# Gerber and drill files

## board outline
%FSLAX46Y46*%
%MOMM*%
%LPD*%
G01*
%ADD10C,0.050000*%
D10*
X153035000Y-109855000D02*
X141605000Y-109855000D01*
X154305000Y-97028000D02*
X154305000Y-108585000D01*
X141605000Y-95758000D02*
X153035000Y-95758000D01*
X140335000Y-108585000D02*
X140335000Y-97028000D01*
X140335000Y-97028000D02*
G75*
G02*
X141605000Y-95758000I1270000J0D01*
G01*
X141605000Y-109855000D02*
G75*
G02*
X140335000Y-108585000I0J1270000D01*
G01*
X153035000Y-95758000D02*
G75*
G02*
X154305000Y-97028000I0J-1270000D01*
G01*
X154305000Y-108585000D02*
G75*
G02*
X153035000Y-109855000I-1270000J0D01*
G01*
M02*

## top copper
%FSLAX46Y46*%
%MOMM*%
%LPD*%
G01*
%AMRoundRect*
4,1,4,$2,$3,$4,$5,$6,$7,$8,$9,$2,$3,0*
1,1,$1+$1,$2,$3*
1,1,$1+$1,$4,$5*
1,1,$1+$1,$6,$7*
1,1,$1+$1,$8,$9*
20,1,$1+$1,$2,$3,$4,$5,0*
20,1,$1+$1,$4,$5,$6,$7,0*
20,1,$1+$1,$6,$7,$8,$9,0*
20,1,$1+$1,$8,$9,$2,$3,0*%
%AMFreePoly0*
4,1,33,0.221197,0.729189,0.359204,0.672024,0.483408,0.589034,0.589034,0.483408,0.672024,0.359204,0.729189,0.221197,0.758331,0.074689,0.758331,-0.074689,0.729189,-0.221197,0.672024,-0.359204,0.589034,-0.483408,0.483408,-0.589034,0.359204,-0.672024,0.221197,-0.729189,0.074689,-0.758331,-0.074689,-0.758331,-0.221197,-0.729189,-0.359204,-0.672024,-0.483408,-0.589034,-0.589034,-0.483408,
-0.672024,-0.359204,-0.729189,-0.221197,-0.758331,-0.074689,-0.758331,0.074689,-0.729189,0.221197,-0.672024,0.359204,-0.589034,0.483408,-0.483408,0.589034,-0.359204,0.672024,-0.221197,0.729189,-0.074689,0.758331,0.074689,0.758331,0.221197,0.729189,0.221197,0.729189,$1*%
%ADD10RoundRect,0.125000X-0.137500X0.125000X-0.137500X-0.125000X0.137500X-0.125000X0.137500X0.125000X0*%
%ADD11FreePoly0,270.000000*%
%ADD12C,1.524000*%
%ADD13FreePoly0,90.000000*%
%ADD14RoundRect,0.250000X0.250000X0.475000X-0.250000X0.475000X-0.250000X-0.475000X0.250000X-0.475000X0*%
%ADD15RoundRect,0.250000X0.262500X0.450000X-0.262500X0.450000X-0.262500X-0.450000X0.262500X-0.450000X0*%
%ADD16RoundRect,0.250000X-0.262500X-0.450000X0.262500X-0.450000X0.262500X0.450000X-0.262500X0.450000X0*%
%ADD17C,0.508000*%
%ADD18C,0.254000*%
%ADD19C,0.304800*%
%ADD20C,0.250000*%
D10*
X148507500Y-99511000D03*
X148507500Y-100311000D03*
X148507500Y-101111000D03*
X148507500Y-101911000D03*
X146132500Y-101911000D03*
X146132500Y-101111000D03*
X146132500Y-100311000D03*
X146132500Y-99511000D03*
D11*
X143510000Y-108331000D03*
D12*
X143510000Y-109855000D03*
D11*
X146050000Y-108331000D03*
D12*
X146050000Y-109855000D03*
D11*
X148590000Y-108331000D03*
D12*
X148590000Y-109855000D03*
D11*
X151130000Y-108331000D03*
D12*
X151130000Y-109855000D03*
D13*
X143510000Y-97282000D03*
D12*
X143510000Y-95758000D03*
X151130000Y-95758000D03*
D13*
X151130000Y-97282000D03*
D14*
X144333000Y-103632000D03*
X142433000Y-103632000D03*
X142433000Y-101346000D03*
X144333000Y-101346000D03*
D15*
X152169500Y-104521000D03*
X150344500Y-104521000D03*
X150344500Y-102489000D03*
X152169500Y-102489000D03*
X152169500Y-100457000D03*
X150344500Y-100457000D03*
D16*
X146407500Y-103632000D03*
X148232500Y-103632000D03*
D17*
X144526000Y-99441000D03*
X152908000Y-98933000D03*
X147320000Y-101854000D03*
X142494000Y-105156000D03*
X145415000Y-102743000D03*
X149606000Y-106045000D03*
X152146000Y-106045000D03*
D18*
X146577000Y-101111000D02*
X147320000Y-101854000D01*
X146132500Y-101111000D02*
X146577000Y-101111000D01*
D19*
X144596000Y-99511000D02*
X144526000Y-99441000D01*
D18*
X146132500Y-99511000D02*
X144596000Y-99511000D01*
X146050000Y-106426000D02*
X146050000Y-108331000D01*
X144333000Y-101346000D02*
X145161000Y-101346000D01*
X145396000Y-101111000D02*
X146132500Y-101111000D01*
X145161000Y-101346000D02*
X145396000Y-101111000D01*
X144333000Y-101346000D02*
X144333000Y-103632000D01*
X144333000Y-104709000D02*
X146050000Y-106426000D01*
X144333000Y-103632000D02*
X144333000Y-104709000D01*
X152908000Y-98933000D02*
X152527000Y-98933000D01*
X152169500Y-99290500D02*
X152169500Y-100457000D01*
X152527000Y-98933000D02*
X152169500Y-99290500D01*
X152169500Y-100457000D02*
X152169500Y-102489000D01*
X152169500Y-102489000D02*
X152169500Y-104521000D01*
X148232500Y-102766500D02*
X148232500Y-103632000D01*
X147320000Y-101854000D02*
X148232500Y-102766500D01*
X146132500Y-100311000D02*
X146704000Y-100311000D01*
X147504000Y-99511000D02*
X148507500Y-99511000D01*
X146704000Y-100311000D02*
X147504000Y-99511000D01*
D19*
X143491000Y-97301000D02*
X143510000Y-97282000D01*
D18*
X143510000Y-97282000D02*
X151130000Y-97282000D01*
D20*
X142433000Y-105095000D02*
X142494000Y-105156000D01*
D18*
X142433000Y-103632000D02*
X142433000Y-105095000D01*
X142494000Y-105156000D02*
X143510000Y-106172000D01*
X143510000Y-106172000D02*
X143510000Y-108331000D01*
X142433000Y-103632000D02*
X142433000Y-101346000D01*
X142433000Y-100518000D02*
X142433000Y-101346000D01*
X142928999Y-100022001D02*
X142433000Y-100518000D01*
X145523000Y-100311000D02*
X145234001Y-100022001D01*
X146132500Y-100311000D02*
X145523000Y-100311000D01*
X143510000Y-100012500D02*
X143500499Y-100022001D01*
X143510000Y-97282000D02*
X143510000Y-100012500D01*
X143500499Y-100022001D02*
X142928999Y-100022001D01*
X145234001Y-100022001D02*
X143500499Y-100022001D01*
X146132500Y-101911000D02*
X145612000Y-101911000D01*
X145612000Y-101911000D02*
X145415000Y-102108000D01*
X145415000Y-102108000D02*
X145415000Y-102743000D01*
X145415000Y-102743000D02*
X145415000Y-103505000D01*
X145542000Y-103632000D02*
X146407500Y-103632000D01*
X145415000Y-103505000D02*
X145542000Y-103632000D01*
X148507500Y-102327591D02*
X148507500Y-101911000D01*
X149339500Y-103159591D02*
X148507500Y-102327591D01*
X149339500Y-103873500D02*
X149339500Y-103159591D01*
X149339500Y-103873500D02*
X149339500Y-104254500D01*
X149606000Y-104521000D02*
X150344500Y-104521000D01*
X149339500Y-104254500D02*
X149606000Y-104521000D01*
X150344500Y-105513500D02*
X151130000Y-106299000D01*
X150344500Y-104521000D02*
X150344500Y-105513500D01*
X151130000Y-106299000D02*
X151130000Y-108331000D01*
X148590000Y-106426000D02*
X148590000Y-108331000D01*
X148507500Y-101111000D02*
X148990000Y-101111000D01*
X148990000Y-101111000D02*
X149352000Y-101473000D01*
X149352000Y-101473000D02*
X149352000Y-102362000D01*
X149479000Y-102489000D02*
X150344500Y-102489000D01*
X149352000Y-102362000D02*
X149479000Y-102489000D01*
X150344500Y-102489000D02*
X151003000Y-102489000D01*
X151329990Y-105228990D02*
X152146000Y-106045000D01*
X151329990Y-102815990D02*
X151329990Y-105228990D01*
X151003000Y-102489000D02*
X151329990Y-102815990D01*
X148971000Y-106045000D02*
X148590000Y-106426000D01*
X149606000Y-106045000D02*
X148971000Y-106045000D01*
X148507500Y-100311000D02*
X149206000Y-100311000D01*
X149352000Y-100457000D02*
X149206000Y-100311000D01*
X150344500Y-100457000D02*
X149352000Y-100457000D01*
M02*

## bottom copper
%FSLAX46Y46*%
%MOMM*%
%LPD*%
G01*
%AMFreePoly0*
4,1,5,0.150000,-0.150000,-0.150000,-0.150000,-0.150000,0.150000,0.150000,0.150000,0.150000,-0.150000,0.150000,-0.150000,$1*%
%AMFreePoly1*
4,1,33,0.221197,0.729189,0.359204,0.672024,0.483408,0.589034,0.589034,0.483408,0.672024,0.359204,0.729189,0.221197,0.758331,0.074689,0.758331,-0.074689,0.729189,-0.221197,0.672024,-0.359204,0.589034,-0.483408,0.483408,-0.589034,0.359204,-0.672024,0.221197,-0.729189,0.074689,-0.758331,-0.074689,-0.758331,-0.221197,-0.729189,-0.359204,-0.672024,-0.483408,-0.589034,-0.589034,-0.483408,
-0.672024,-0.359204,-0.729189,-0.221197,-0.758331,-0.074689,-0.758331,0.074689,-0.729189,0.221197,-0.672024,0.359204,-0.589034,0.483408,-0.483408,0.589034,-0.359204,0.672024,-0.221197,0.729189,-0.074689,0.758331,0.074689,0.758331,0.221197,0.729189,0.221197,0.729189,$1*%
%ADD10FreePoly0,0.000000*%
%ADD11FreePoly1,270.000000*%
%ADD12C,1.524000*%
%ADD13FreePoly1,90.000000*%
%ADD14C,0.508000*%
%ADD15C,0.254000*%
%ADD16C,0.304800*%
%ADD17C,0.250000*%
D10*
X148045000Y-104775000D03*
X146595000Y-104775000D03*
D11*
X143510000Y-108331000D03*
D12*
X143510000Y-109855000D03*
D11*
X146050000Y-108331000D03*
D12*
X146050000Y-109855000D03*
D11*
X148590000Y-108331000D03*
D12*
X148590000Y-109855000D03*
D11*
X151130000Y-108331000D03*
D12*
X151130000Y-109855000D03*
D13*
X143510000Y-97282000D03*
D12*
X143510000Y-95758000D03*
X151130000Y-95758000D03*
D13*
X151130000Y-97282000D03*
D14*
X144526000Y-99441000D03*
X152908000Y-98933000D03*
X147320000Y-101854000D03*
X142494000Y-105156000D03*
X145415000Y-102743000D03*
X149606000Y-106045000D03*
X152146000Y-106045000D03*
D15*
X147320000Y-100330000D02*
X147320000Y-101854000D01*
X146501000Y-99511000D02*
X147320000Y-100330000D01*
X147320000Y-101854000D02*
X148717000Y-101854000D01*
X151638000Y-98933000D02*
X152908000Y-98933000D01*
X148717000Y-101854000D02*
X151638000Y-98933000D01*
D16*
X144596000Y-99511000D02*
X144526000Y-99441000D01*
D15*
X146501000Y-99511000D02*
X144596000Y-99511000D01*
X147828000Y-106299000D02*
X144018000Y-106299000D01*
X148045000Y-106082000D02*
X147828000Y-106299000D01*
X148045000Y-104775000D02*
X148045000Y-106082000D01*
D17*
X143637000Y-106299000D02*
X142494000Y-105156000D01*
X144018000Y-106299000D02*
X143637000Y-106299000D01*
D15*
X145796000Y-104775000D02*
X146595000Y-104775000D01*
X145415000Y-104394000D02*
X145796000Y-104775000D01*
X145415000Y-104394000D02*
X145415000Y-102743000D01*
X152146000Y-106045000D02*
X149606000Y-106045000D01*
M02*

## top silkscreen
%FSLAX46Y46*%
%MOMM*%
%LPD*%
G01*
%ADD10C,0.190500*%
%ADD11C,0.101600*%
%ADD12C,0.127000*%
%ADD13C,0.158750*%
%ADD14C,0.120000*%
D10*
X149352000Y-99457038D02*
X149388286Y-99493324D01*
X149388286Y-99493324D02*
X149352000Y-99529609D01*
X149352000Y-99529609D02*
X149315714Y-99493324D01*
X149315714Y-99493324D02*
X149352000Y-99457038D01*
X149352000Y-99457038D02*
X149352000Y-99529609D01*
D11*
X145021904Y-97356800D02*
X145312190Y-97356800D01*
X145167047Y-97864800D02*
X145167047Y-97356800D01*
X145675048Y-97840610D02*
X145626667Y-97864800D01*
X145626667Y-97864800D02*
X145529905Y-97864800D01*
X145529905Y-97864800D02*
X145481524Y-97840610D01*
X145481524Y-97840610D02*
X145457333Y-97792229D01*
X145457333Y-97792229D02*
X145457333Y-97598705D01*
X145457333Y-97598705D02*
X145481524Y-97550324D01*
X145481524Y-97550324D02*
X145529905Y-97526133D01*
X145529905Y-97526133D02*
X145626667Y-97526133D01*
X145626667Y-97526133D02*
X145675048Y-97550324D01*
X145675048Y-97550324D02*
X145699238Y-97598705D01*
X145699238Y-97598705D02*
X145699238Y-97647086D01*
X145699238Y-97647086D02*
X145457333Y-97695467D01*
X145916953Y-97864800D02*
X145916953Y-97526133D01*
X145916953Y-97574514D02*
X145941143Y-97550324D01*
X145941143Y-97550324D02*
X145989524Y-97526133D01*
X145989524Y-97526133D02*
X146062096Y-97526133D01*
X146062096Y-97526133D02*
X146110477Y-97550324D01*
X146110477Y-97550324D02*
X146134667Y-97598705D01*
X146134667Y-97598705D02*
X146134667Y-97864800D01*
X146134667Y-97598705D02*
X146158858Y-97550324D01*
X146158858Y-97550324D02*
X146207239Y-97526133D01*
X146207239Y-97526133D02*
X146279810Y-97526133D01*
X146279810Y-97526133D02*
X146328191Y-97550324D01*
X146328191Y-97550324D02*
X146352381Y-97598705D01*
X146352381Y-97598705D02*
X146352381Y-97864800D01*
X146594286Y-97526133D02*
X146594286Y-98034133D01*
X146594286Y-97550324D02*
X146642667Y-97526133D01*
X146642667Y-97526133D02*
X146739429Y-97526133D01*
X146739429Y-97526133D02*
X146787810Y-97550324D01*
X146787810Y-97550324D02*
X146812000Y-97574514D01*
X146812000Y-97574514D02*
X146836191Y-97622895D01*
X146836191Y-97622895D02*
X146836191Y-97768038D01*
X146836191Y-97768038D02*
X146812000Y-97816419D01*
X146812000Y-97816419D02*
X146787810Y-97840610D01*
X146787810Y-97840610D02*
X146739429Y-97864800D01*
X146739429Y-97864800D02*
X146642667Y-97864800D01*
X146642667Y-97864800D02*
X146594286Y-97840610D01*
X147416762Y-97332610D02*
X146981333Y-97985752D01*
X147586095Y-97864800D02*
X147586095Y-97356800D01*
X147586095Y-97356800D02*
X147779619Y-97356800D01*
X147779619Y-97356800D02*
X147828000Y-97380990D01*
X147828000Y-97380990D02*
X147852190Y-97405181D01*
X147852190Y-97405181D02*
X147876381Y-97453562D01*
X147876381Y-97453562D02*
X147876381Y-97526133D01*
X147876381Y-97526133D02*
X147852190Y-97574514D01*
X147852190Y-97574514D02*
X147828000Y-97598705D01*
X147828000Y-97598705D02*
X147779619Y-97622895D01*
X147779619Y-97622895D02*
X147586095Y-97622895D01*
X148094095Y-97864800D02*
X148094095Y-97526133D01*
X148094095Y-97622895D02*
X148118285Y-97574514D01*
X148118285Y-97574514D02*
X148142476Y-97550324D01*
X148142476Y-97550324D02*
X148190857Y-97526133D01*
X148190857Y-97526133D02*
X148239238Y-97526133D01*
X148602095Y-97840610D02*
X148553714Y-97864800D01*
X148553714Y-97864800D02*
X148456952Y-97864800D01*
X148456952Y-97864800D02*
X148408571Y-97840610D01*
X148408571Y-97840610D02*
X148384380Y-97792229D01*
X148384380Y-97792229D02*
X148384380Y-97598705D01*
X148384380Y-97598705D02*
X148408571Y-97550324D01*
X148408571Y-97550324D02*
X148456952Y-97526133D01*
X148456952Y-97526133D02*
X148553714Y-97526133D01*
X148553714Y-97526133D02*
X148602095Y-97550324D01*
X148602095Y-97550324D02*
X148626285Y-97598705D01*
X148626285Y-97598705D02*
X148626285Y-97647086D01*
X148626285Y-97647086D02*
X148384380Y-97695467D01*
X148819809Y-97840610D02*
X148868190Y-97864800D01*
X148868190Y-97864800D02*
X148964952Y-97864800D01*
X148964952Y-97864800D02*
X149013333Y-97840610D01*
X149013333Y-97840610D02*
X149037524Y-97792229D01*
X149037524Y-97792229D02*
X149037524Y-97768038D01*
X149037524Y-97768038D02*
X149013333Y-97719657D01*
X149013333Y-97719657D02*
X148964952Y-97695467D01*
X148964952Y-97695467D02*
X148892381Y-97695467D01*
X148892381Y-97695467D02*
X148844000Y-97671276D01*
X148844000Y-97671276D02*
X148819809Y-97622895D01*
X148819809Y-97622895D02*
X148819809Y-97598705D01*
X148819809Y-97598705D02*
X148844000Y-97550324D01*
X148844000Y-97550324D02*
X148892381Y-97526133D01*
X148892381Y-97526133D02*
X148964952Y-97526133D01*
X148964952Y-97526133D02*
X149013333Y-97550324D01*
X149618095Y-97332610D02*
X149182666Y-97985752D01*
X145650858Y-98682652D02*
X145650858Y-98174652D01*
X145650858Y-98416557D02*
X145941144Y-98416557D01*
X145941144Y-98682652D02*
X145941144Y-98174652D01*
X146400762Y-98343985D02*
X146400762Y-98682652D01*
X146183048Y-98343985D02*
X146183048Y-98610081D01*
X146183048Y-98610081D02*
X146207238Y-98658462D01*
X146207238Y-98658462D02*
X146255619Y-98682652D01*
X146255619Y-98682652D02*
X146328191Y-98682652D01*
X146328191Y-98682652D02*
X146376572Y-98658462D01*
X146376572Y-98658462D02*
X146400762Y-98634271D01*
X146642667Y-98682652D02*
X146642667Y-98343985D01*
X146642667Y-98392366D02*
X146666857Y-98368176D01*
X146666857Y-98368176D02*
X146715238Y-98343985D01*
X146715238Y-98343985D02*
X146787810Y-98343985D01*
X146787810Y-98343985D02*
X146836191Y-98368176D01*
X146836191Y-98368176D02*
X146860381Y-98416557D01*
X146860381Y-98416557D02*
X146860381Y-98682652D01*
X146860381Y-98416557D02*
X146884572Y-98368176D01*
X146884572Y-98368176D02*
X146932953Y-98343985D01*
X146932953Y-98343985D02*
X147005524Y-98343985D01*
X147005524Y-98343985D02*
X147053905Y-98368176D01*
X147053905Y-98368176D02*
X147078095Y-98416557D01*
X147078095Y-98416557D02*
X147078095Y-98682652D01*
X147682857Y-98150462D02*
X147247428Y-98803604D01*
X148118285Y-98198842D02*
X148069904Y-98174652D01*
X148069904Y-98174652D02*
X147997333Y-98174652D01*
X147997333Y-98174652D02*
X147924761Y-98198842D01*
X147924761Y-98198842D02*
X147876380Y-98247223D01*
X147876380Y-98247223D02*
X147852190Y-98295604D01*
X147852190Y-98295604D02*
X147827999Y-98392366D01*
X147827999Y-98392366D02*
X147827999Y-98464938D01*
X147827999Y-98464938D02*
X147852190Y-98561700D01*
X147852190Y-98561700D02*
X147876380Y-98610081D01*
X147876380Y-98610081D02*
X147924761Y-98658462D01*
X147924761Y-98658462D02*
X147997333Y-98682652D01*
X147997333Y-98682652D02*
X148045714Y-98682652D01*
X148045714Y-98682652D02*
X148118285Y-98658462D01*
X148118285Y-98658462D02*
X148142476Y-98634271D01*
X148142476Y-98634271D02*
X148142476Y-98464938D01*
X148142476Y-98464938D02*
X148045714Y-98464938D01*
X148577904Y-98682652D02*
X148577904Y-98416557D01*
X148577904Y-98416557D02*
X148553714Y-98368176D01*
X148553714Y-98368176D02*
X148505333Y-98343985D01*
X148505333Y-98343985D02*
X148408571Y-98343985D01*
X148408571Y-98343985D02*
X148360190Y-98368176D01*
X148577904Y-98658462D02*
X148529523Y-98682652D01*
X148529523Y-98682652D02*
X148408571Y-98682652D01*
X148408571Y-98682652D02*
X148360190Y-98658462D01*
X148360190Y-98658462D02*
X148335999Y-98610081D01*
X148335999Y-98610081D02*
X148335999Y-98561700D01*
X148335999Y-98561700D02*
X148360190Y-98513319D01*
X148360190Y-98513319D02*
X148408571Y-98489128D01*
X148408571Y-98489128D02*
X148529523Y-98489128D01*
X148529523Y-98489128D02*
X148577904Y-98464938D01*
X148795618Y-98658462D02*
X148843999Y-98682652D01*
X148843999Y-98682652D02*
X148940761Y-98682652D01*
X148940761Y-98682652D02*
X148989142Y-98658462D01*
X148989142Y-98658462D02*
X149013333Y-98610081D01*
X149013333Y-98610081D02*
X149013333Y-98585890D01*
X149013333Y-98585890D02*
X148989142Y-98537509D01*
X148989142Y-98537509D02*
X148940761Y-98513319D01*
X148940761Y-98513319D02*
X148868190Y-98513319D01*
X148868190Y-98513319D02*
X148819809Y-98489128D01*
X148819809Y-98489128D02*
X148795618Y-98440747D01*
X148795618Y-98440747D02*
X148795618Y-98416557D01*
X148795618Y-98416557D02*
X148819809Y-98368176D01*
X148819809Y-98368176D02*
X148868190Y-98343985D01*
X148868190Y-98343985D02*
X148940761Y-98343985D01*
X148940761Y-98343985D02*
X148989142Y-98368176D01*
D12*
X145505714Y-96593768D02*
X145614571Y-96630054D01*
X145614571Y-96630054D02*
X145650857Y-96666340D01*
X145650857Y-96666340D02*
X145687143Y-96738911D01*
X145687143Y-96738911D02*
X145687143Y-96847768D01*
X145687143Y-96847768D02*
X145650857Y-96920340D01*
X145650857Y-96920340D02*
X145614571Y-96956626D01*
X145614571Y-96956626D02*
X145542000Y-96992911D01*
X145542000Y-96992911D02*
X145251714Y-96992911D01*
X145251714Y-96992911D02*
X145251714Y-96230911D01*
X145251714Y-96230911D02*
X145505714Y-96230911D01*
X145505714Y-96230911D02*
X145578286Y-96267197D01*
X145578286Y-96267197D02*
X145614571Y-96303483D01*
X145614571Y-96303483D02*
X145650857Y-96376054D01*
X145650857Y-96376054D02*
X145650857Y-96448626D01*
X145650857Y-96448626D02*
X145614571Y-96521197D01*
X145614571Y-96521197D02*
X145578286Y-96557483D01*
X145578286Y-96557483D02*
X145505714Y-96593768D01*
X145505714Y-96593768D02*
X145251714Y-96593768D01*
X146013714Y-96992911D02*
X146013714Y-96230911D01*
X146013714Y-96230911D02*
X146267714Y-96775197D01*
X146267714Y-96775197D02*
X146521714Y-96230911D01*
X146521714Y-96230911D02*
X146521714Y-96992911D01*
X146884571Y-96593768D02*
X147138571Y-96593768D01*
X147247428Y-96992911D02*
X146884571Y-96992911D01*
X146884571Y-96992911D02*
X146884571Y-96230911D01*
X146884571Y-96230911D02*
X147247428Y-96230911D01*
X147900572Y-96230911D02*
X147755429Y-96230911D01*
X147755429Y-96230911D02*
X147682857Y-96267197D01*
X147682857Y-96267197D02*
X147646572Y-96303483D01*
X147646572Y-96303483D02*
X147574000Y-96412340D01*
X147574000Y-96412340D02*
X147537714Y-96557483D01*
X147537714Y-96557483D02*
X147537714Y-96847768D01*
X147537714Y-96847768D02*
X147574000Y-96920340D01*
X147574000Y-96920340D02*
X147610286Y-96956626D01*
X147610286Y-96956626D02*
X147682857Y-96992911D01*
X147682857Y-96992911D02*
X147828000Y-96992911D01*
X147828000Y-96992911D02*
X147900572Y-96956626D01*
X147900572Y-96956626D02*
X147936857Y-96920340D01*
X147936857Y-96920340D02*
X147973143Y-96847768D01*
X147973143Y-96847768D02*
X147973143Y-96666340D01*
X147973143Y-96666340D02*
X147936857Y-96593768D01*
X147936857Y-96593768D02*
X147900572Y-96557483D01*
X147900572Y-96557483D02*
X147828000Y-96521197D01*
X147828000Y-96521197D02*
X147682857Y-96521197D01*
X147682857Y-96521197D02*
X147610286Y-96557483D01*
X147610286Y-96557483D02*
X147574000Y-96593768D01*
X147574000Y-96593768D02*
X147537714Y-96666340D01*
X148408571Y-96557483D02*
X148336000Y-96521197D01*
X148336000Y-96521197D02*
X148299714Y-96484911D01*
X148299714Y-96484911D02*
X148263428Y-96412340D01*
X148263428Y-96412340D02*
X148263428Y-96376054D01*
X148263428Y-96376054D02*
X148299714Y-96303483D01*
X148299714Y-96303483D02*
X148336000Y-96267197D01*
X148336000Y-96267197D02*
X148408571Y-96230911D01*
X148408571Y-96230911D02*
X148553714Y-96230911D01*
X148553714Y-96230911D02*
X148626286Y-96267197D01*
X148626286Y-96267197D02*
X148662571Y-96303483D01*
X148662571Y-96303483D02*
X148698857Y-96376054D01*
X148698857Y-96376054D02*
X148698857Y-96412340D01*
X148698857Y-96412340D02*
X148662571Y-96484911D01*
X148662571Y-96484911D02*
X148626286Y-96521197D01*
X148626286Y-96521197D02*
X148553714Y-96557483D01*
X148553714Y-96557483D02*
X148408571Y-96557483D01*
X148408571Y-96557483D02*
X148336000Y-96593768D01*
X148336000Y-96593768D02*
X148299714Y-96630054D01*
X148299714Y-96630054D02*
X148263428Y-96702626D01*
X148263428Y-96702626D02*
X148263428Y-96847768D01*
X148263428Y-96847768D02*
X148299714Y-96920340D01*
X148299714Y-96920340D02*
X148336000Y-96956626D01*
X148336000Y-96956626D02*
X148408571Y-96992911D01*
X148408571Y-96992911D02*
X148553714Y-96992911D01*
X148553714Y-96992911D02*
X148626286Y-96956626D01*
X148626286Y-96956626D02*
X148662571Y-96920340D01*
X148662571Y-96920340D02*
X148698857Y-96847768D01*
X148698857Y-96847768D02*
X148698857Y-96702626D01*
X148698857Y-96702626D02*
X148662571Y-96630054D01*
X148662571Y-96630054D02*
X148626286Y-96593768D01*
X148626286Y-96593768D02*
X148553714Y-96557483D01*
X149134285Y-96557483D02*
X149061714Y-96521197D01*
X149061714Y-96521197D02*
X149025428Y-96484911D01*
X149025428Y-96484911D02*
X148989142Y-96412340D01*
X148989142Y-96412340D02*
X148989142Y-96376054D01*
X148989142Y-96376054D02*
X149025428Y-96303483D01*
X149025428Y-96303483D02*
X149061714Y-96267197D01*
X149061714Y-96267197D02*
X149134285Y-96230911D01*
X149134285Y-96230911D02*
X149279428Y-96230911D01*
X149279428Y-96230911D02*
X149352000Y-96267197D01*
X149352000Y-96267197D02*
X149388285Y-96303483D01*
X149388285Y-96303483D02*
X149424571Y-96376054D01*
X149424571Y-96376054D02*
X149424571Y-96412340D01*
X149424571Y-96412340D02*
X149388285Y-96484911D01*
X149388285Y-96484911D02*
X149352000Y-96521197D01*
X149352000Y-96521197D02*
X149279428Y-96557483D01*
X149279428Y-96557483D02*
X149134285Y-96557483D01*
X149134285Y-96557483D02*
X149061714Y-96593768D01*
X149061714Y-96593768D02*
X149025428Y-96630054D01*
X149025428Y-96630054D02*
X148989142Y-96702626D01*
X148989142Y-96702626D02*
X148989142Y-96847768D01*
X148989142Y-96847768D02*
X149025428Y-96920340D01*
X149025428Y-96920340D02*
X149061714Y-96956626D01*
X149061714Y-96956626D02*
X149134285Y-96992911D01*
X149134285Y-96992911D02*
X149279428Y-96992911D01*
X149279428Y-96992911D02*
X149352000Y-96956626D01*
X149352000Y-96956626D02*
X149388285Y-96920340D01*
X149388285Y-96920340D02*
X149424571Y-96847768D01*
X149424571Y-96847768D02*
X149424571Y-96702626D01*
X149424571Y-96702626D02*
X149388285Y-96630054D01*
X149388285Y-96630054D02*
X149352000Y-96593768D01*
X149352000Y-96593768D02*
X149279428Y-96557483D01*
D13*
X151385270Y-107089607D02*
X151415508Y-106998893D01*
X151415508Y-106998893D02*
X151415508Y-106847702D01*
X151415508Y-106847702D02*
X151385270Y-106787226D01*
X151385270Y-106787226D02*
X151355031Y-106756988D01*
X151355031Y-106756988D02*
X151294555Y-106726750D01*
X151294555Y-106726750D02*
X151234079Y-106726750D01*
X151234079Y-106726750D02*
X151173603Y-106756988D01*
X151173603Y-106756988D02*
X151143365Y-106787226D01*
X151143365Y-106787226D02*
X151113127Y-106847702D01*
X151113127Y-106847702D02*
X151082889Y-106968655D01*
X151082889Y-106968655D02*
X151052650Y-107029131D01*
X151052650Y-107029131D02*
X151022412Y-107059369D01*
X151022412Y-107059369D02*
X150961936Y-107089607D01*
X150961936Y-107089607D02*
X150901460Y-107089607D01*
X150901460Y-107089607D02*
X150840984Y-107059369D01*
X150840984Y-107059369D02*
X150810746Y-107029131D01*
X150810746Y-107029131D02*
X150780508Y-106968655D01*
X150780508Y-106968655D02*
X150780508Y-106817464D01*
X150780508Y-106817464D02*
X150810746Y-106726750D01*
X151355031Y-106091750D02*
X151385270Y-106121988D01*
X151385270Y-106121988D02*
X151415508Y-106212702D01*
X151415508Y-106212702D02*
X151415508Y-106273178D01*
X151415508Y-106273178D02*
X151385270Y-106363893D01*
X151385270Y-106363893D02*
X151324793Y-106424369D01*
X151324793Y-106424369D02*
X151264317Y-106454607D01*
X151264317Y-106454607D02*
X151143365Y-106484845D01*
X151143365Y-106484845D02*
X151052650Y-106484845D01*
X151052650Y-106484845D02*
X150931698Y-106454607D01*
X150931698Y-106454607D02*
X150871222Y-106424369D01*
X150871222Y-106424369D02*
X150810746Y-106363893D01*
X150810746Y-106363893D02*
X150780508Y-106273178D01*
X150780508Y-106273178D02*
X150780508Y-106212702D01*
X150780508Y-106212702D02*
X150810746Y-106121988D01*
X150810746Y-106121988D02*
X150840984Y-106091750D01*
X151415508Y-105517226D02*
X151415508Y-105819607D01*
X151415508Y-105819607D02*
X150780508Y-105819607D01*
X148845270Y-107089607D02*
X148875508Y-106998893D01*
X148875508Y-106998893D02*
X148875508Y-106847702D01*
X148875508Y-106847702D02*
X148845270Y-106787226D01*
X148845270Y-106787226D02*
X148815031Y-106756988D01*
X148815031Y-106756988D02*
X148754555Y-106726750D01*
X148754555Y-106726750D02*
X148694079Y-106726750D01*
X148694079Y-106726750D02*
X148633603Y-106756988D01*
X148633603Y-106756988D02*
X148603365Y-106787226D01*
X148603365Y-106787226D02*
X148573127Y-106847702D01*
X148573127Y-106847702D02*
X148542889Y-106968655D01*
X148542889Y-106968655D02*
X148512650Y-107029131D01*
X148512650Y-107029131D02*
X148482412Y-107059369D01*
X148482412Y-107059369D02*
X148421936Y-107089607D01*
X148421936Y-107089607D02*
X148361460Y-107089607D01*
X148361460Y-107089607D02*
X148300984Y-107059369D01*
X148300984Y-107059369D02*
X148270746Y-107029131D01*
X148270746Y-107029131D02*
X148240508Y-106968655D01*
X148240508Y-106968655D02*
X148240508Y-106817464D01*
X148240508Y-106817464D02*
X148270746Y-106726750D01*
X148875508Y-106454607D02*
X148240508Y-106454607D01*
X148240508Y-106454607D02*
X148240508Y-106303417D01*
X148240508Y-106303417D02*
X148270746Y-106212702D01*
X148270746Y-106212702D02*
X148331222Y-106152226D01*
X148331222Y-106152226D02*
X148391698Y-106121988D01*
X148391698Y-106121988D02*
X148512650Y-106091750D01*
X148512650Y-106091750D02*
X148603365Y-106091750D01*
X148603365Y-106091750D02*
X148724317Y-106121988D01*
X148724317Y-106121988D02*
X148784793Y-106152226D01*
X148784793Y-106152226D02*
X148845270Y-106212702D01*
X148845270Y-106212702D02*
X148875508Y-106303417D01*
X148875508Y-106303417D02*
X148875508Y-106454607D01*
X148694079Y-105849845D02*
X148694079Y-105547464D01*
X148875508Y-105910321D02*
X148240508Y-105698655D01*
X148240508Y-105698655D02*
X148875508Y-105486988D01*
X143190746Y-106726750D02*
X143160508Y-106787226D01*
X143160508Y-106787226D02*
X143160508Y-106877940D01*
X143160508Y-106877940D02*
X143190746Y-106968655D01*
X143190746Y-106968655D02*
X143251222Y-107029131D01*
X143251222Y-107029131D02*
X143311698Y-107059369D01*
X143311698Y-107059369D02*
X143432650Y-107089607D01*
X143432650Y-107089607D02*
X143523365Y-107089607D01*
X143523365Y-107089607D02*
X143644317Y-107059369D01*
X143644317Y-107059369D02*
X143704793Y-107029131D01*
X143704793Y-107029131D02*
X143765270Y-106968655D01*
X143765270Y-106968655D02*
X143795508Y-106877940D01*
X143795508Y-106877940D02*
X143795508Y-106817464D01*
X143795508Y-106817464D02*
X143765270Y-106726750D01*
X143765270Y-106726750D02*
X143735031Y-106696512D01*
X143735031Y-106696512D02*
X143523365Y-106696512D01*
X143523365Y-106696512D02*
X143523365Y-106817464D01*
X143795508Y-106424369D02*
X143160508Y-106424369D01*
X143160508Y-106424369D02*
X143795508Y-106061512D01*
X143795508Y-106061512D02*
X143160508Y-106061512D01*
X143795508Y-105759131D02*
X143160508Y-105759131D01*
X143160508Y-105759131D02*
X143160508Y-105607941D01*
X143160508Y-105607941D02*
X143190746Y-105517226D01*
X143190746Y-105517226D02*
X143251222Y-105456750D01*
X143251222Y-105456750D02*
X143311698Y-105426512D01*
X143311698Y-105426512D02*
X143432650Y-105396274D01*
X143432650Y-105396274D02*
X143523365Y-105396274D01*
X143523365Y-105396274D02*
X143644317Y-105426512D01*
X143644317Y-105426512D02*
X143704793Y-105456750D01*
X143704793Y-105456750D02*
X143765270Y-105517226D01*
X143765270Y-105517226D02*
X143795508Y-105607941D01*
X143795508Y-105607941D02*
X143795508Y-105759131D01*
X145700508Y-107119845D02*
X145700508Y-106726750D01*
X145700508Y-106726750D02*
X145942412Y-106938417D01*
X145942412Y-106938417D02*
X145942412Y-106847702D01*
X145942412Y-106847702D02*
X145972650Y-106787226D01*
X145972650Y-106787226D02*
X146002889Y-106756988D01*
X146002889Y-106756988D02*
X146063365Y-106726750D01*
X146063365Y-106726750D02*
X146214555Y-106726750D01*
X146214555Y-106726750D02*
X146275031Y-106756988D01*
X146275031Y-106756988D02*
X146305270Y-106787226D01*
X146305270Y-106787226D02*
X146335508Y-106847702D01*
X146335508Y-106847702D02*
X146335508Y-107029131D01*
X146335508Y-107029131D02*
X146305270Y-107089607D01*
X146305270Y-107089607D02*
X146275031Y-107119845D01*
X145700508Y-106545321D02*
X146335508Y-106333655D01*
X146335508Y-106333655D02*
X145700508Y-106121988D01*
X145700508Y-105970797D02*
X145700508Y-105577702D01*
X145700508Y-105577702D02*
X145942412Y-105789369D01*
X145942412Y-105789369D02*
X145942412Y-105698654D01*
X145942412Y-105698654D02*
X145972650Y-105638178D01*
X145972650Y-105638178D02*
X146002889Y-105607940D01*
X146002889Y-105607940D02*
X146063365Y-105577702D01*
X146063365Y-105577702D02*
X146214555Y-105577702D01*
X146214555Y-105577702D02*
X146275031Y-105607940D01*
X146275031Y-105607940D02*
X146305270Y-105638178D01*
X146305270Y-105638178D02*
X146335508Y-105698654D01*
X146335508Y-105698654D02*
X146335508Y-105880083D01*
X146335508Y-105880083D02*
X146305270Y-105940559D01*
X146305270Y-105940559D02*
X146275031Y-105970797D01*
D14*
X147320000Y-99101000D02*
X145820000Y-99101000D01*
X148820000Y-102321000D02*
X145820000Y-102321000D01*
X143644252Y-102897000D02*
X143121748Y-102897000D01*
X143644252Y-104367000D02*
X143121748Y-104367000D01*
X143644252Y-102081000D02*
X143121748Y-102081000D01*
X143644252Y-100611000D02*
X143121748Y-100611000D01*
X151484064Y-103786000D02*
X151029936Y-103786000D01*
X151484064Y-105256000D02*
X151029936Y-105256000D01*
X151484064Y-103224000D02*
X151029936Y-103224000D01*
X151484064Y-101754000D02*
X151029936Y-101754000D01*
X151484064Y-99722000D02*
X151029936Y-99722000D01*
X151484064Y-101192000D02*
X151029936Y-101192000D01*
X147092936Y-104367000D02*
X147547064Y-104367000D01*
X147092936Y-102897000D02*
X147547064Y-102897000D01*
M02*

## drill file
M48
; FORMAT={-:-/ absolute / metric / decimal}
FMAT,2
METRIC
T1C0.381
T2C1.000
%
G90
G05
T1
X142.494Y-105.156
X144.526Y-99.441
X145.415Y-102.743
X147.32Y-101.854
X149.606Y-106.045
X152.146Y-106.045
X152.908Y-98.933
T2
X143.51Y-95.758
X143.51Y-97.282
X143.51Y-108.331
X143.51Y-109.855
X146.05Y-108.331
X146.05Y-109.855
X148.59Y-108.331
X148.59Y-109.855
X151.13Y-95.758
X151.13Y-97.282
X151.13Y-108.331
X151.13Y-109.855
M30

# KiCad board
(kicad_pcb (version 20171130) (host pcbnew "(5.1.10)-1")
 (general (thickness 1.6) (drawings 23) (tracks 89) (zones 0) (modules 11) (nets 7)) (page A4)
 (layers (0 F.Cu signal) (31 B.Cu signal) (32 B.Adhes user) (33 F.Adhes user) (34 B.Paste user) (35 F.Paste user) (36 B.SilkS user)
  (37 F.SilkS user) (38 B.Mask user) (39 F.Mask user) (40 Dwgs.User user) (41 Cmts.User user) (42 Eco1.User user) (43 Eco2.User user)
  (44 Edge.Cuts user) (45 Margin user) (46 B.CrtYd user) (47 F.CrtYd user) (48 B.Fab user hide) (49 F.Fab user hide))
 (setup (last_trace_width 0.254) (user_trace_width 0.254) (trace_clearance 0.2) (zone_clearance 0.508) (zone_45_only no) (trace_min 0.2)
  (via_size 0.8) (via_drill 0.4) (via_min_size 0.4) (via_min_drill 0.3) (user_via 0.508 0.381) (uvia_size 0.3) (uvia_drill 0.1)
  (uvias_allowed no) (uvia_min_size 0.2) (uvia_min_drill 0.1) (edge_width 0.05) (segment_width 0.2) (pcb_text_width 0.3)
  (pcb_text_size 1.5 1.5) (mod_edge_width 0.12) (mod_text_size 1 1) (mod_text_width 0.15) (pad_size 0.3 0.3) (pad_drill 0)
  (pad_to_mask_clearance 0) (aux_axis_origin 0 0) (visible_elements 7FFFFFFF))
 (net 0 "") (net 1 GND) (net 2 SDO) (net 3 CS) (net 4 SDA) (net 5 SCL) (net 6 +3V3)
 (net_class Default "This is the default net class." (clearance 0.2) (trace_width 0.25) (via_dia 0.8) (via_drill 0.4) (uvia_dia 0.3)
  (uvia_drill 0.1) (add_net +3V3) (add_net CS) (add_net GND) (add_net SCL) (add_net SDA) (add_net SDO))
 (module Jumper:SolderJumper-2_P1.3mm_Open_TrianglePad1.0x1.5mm (layer B.Cu) (at 147.32 104.775)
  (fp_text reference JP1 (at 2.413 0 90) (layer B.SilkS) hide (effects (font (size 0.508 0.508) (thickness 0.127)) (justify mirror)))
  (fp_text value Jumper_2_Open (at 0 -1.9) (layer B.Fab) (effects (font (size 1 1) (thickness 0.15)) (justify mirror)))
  (pad 2 smd custom (at 0.725 0) (size 0.3 0.3) (layers B.Cu B.Mask) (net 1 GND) (zone_connect 2)
   (options (clearance outline) (anchor rect)) (primitives))
  (pad 1 smd custom (at -0.725 0) (size 0.3 0.3) (layers B.Cu B.Mask) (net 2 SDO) (zone_connect 2)
   (options (clearance outline) (anchor rect)) (primitives)))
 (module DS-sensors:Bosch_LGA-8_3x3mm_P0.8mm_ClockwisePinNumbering (layer F.Cu) (at 147.32 100.711 270)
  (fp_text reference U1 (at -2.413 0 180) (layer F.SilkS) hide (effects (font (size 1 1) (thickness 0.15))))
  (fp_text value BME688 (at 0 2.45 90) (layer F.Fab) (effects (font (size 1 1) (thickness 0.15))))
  (fp_line (start -1.61 0) (end -1.61 1.5) (layer F.SilkS) (width 0.12))
  (fp_line (start 1.61 -1.5) (end 1.61 1.5) (layer F.SilkS) (width 0.12))
  (pad 1 smd roundrect (at -1.2 -1.1875 270) (size 0.5 0.525) (layers F.Cu F.Paste F.Mask) (roundrect_rratio 0.25) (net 1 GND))
  (pad 2 smd roundrect (at -0.4 -1.1875 270) (size 0.5 0.525) (layers F.Cu F.Paste F.Mask) (roundrect_rratio 0.25) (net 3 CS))
  (pad 3 smd roundrect (at 0.4 -1.1875 270) (size 0.5 0.525) (layers F.Cu F.Paste F.Mask) (roundrect_rratio 0.25) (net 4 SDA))
  (pad 4 smd roundrect (at 1.2 -1.1875 270) (size 0.5 0.525) (layers F.Cu F.Paste F.Mask) (roundrect_rratio 0.25) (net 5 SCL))
  (pad 5 smd roundrect (at 1.2 1.1875 270) (size 0.5 0.525) (layers F.Cu F.Paste F.Mask) (roundrect_rratio 0.25) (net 2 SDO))
  (pad 6 smd roundrect (at 0.4 1.1875 270) (size 0.5 0.525) (layers F.Cu F.Paste F.Mask) (roundrect_rratio 0.25) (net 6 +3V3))
  (pad 7 smd roundrect (at -0.4 1.1875 270) (size 0.5 0.525) (layers F.Cu F.Paste F.Mask) (roundrect_rratio 0.25) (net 1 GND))
  (pad 8 smd roundrect (at -1.2 1.1875 270) (size 0.5 0.525) (layers F.Cu F.Paste F.Mask) (roundrect_rratio 0.25) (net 6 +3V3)))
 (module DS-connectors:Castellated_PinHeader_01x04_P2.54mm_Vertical (layer B.Cu) (at 140.97 108.331 270)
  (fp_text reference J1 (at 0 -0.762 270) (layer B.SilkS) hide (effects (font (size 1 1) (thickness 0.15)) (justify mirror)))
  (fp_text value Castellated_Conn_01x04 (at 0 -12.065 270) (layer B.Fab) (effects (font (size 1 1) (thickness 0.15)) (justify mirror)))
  (pad 1 thru_hole custom (at 0 -2.54 270) (size 1.524 1.524) (drill 1) (layers *.Cu *.Mask) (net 1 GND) (zone_connect 0)
   (options (clearance outline) (anchor circle)) (primitives))
  (pad 1 thru_hole circle (at 1.524 -2.54 270) (size 1.524 1.524) (drill 1) (layers *.Cu *.Mask) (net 1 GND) (zone_connect 0))
  (pad 2 thru_hole custom (at 0 -5.08 270) (size 1.524 1.524) (drill 1) (layers *.Cu *.Mask) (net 6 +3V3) (zone_connect 0)
   (options (clearance outline) (anchor circle)) (primitives))
  (pad 2 thru_hole circle (at 1.524 -5.08 270) (size 1.524 1.524) (drill 1) (layers *.Cu *.Mask) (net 6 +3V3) (zone_connect 0))
  (pad 3 thru_hole custom (at 0 -7.62 270) (size 1.524 1.524) (drill 1) (layers *.Cu *.Mask) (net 4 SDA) (zone_connect 0)
   (options (clearance outline) (anchor circle)) (primitives))
  (pad 3 thru_hole circle (at 1.524 -7.62 270) (size 1.524 1.524) (drill 1) (layers *.Cu *.Mask) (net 4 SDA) (zone_connect 0))
  (pad 4 thru_hole custom (at 0 -10.16 270) (size 1.524 1.524) (drill 1) (layers *.Cu *.Mask) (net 5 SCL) (zone_connect 0)
   (options (clearance outline) (anchor circle)) (primitives))
  (pad 4 thru_hole circle (at 1.524 -10.16 270) (size 1.524 1.524) (drill 1) (layers *.Cu *.Mask) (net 5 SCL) (zone_connect 0)))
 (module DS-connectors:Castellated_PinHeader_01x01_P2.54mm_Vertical (layer F.Cu) (at 141.478 97.282 90)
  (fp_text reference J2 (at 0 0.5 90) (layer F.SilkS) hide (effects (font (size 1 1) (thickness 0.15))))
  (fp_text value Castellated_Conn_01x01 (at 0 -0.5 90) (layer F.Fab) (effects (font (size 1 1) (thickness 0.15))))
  (pad 1 thru_hole custom (at 0 2.032 90) (size 1.524 1.524) (drill 1) (layers *.Cu *.Mask) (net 1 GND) (zone_connect 0)
   (options (clearance outline) (anchor circle)) (primitives))
  (pad 1 thru_hole circle (at 1.524 2.032 90) (size 1.524 1.524) (drill 1) (layers *.Cu *.Mask) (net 1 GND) (zone_connect 0)))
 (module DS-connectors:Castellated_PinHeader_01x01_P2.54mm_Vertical (layer F.Cu) (at 149.098 97.282 90)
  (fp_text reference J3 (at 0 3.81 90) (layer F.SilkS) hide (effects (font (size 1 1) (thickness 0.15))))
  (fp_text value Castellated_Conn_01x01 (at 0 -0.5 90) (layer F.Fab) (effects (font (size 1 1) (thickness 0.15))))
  (pad 1 thru_hole circle (at 1.524 2.032 90) (size 1.524 1.524) (drill 1) (layers *.Cu *.Mask) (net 1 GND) (zone_connect 0))
  (pad 1 thru_hole custom (at 0 2.032 90) (size 1.524 1.524) (drill 1) (layers *.Cu *.Mask) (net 1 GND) (zone_connect 0)
   (options (clearance outline) (anchor circle)) (primitives)))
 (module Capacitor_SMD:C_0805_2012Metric (layer F.Cu) (at 143.383 103.632 180)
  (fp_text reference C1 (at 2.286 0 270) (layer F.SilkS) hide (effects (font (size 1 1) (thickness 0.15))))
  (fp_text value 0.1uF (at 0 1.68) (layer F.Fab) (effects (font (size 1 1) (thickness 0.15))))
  (fp_line (start -0.261252 0.735) (end 0.261252 0.735) (layer F.SilkS) (width 0.12))
  (fp_line (start -0.261252 -0.735) (end 0.261252 -0.735) (layer F.SilkS) (width 0.12))
  (pad 1 smd roundrect (at -0.95 0 180) (size 1 1.45) (layers F.Cu F.Paste F.Mask) (roundrect_rratio 0.25) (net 6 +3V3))
  (pad 2 smd roundrect (at 0.95 0 180) (size 1 1.45) (layers F.Cu F.Paste F.Mask) (roundrect_rratio 0.25) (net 1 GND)))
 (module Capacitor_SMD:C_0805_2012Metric (layer F.Cu) (at 143.383 101.346 180)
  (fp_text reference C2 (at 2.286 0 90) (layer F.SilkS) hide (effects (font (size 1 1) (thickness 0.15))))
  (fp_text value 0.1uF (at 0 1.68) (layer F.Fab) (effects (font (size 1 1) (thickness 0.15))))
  (fp_line (start -0.261252 -0.735) (end 0.261252 -0.735) (layer F.SilkS) (width 0.12))
  (fp_line (start -0.261252 0.735) (end 0.261252 0.735) (layer F.SilkS) (width 0.12))
  (pad 2 smd roundrect (at 0.95 0 180) (size 1 1.45) (layers F.Cu F.Paste F.Mask) (roundrect_rratio 0.25) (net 1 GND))
  (pad 1 smd roundrect (at -0.95 0 180) (size 1 1.45) (layers F.Cu F.Paste F.Mask) (roundrect_rratio 0.25) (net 6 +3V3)))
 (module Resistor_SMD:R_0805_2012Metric (layer F.Cu) (at 151.257 104.521 180)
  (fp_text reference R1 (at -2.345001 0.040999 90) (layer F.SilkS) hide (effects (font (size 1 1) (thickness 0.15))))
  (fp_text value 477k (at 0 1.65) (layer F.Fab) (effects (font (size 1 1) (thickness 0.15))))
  (fp_line (start -0.227064 0.735) (end 0.227064 0.735) (layer F.SilkS) (width 0.12))
  (fp_line (start -0.227064 -0.735) (end 0.227064 -0.735) (layer F.SilkS) (width 0.12))
  (pad 1 smd roundrect (at -0.9125 0 180) (size 1.025 1.4) (layers F.Cu F.Paste F.Mask) (roundrect_rratio 0.243902) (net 6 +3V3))
  (pad 2 smd roundrect (at 0.9125 0 180) (size 1.025 1.4) (layers F.Cu F.Paste F.Mask) (roundrect_rratio 0.243902) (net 5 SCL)))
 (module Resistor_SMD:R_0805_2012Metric (layer F.Cu) (at 151.257 102.489 180)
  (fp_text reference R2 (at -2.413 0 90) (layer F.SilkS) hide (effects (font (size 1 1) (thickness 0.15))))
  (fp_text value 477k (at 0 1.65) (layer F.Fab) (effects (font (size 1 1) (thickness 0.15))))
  (fp_line (start -0.227064 -0.735) (end 0.227064 -0.735) (layer F.SilkS) (width 0.12))
  (fp_line (start -0.227064 0.735) (end 0.227064 0.735) (layer F.SilkS) (width 0.12))
  (pad 2 smd roundrect (at 0.9125 0 180) (size 1.025 1.4) (layers F.Cu F.Paste F.Mask) (roundrect_rratio 0.243902) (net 4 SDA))
  (pad 1 smd roundrect (at -0.9125 0 180) (size 1.025 1.4) (layers F.Cu F.Paste F.Mask) (roundrect_rratio 0.243902) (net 6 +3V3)))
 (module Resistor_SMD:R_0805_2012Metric (layer F.Cu) (at 151.257 100.457 180)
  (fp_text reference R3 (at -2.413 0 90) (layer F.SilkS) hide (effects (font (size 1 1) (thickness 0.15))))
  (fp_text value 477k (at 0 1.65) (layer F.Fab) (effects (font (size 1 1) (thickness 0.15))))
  (fp_line (start -0.227064 0.735) (end 0.227064 0.735) (layer F.SilkS) (width 0.12))
  (fp_line (start -0.227064 -0.735) (end 0.227064 -0.735) (layer F.SilkS) (width 0.12))
  (pad 1 smd roundrect (at -0.9125 0 180) (size 1.025 1.4) (layers F.Cu F.Paste F.Mask) (roundrect_rratio 0.243902) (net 6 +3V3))
  (pad 2 smd roundrect (at 0.9125 0 180) (size 1.025 1.4) (layers F.Cu F.Paste F.Mask) (roundrect_rratio 0.243902) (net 3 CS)))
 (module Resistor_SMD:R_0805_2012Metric (layer F.Cu) (at 147.32 103.632)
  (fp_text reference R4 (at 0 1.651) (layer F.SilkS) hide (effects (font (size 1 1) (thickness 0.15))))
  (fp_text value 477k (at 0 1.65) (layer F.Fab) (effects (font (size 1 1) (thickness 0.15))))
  (fp_line (start -0.227064 0.735) (end 0.227064 0.735) (layer F.SilkS) (width 0.12))
  (fp_line (start -0.227064 -0.735) (end 0.227064 -0.735) (layer F.SilkS) (width 0.12))
  (pad 1 smd roundrect (at -0.9125 0) (size 1.025 1.4) (layers F.Cu F.Paste F.Mask) (roundrect_rratio 0.243902) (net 2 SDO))
  (pad 2 smd roundrect (at 0.9125 0) (size 1.025 1.4) (layers F.Cu F.Paste F.Mask) (roundrect_rratio 0.243902) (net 6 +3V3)))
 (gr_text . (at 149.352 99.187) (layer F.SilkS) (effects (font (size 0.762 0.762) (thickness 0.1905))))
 (gr_line (start 153.035 109.855) (end 141.605 109.855) (layer Edge.Cuts) (width 0.05))
 (gr_line (start 154.305 97.028) (end 154.305 108.585) (layer Edge.Cuts) (width 0.05))
 (gr_line (start 141.605 95.758) (end 153.035 95.758) (layer Edge.Cuts) (width 0.05))
 (gr_line (start 140.335 108.585) (end 140.335 97.028) (layer Edge.Cuts) (width 0.05))
 (gr_arc (start 141.605 97.028) (end 141.605 95.758) (angle -90) (layer Edge.Cuts) (width 0.05))
 (gr_arc (start 141.605 108.585) (end 140.335 108.585) (angle -90) (layer Edge.Cuts) (width 0.05))
 (gr_arc (start 153.035 97.028) (end 154.305 97.028) (angle -90) (layer Edge.Cuts) (width 0.05))
 (gr_arc (start 153.035 108.585) (end 153.035 109.855) (angle -90) (layer Edge.Cuts) (width 0.05))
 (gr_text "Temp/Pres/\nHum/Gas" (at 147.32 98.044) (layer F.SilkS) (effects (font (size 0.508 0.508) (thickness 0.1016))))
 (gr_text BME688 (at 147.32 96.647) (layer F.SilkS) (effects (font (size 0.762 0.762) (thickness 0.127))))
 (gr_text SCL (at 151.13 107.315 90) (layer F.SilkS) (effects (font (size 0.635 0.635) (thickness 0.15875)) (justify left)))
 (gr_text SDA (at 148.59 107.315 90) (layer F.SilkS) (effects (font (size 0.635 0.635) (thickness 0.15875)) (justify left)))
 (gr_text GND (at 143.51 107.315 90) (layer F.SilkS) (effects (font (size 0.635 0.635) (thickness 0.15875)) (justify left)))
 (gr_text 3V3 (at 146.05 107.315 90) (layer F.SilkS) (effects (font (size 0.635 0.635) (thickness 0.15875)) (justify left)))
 (via (at 144.526 99.441) (size 0.508) (drill 0.381) (layers F.Cu B.Cu) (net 6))
 (via (at 152.908 98.933) (size 0.508) (drill 0.381) (layers F.Cu B.Cu) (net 6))
 (via (at 147.32 101.854) (size 0.508) (drill 0.381) (layers F.Cu B.Cu) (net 6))
 (segment (start 146.577 101.111) (end 147.32 101.854) (width 0.254) (layer F.Cu) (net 6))
 (segment (start 146.1325 101.111) (end 146.577 101.111) (width 0.254) (layer F.Cu) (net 6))
 (segment (start 147.32 100.33) (end 147.32 101.854) (width 0.254) (layer B.Cu) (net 6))
 (segment (start 146.501 99.511) (end 147.32 100.33) (width 0.254) (layer B.Cu) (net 6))
 (segment (start 147.32 101.854) (end 148.717 101.854) (width 0.254) (layer B.Cu) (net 6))
 (segment (start 151.638 98.933) (end 152.908 98.933) (width 0.254) (layer B.Cu) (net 6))
 (segment (start 148.717 101.854) (end 151.638 98.933) (width 0.254) (layer B.Cu) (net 6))
 (segment (start 144.596 99.511) (end 144.526 99.441) (width 0.3048) (layer B.Cu) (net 6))
 (segment (start 146.501 99.511) (end 144.596 99.511) (width 0.254) (layer B.Cu) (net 6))
 (segment (start 144.596 99.511) (end 144.526 99.441) (width 0.3048) (layer F.Cu) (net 6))
 (segment (start 146.1325 99.511) (end 144.596 99.511) (width 0.254) (layer F.Cu) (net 6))
 (segment (start 146.05 106.426) (end 146.05 108.331) (width 0.254) (layer F.Cu) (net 6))
 (segment (start 144.333 101.346) (end 145.161 101.346) (width 0.254) (layer F.Cu) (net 6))
 (segment (start 145.396 101.111) (end 146.1325 101.111) (width 0.254) (layer F.Cu) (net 6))
 (segment (start 145.161 101.346) (end 145.396 101.111) (width 0.254) (layer F.Cu) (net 6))
 (segment (start 144.333 101.346) (end 144.333 103.632) (width 0.254) (layer F.Cu) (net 6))
 (segment (start 144.333 104.709) (end 146.05 106.426) (width 0.254) (layer F.Cu) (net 6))
 (segment (start 144.333 103.632) (end 144.333 104.709) (width 0.254) (layer F.Cu) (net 6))
 (segment (start 152.908 98.933) (end 152.527 98.933) (width 0.254) (layer F.Cu) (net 6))
 (segment (start 152.1695 99.2905) (end 152.1695 100.457) (width 0.254) (layer F.Cu) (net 6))
 (segment (start 152.527 98.933) (end 152.1695 99.2905) (width 0.254) (layer F.Cu) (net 6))
 (segment (start 152.1695 100.457) (end 152.1695 102.489) (width 0.254) (layer F.Cu) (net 6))
 (segment (start 152.1695 102.489) (end 152.1695 104.521) (width 0.254) (layer F.Cu) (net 6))
 (segment (start 148.2325 102.7665) (end 148.2325 103.632) (width 0.254) (layer F.Cu) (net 6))
 (segment (start 147.32 101.854) (end 148.2325 102.7665) (width 0.254) (layer F.Cu) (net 6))
 (via (at 142.494 105.156) (size 0.508) (drill 0.381) (layers F.Cu B.Cu) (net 1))
 (segment (start 146.1325 100.311) (end 146.704 100.311) (width 0.254) (layer F.Cu) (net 1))
 (segment (start 147.504 99.511) (end 148.5075 99.511) (width 0.254) (layer F.Cu) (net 1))
 (segment (start 146.704 100.311) (end 147.504 99.511) (width 0.254) (layer F.Cu) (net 1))
 (segment (start 147.828 106.299) (end 144.018 106.299) (width 0.254) (layer B.Cu) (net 1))
 (segment (start 148.045 106.082) (end 147.828 106.299) (width 0.254) (layer B.Cu) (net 1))
 (segment (start 148.045 104.775) (end 148.045 106.082) (width 0.254) (layer B.Cu) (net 1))
 (segment (start 143.491 97.301) (end 143.51 97.282) (width 0.3048) (layer F.Cu) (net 1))
 (segment (start 143.51 97.282) (end 151.13 97.282) (width 0.254) (layer F.Cu) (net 1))
 (segment (start 142.433 105.095) (end 142.494 105.156) (width 0.25) (layer F.Cu) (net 1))
 (segment (start 142.433 103.632) (end 142.433 105.095) (width 0.254) (layer F.Cu) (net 1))
 (segment (start 142.494 105.156) (end 143.51 106.172) (width 0.254) (layer F.Cu) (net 1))
 (segment (start 143.51 106.172) (end 143.51 108.331) (width 0.254) (layer F.Cu) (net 1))
 (segment (start 143.637 106.299) (end 142.494 105.156) (width 0.25) (layer B.Cu) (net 1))
 (segment (start 144.018 106.299) (end 143.637 106.299) (width 0.25) (layer B.Cu) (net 1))
 (segment (start 142.433 103.632) (end 142.433 101.346) (width 0.254) (layer F.Cu) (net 1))
 (segment (start 142.433 100.518) (end 142.433 101.346) (width 0.254) (layer F.Cu) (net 1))
 (segment (start 142.928999 100.022001) (end 142.433 100.518) (width 0.254) (layer F.Cu) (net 1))
 (segment (start 145.523 100.311) (end 145.234001 100.022001) (width 0.254) (layer F.Cu) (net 1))
 (segment (start 146.1325 100.311) (end 145.523 100.311) (width 0.254) (layer F.Cu) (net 1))
 (segment (start 143.51 100.0125) (end 143.500499 100.022001) (width 0.254) (layer F.Cu) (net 1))
 (segment (start 143.51 97.282) (end 143.51 100.0125) (width 0.254) (layer F.Cu) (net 1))
 (segment (start 143.500499 100.022001) (end 142.928999 100.022001) (width 0.254) (layer F.Cu) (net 1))
 (segment (start 145.234001 100.022001) (end 143.500499 100.022001) (width 0.254) (layer F.Cu) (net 1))
 (via (at 145.415 102.743) (size 0.508) (drill 0.381) (layers F.Cu B.Cu) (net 2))
 (segment (start 146.1325 101.911) (end 145.612 101.911) (width 0.254) (layer F.Cu) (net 2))
 (segment (start 145.612 101.911) (end 145.415 102.108) (width 0.254) (layer F.Cu) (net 2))
 (segment (start 145.796 104.775) (end 146.595 104.775) (width 0.254) (layer B.Cu) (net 2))
 (segment (start 145.415 104.394) (end 145.796 104.775) (width 0.254) (layer B.Cu) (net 2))
 (segment (start 145.415 102.108) (end 145.415 102.743) (width 0.254) (layer F.Cu) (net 2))
 (segment (start 145.415 102.743) (end 145.415 103.505) (width 0.254) (layer F.Cu) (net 2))
 (segment (start 145.542 103.632) (end 146.4075 103.632) (width 0.254) (layer F.Cu) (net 2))
 (segment (start 145.415 103.505) (end 145.542 103.632) (width 0.254) (layer F.Cu) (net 2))
 (segment (start 145.415 104.394) (end 145.415 102.743) (width 0.254) (layer B.Cu) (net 2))
 (segment (start 148.5075 102.327591) (end 148.5075 101.911) (width 0.254) (layer F.Cu) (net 5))
 (segment (start 149.3395 103.159591) (end 148.5075 102.327591) (width 0.254) (layer F.Cu) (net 5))
 (segment (start 149.3395 103.8735) (end 149.3395 103.159591) (width 0.254) (layer F.Cu) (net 5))
 (segment (start 149.3395 103.8735) (end 149.3395 104.2545) (width 0.254) (layer F.Cu) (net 5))
 (segment (start 149.606 104.521) (end 150.3445 104.521) (width 0.254) (layer F.Cu) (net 5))
 (segment (start 149.3395 104.2545) (end 149.606 104.521) (width 0.254) (layer F.Cu) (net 5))
 (segment (start 150.3445 105.5135) (end 151.13 106.299) (width 0.254) (layer F.Cu) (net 5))
 (segment (start 150.3445 104.521) (end 150.3445 105.5135) (width 0.254) (layer F.Cu) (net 5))
 (segment (start 151.13 106.299) (end 151.13 108.331) (width 0.254) (layer F.Cu) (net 5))
 (via (at 149.606 106.045) (size 0.508) (drill 0.381) (layers F.Cu B.Cu) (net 4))
 (via (at 152.146 106.045) (size 0.508) (drill 0.381) (layers F.Cu B.Cu) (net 4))
 (segment (start 148.59 106.426) (end 148.59 108.331) (width 0.254) (layer F.Cu) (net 4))
 (segment (start 148.5075 101.111) (end 148.99 101.111) (width 0.254) (layer F.Cu) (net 4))
 (segment (start 148.99 101.111) (end 149.352 101.473) (width 0.254) (layer F.Cu) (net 4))
 (segment (start 149.352 101.473) (end 149.352 102.362) (width 0.254) (layer F.Cu) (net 4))
 (segment (start 149.479 102.489) (end 150.3445 102.489) (width 0.254) (layer F.Cu) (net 4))
 (segment (start 149.352 102.362) (end 149.479 102.489) (width 0.254) (layer F.Cu) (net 4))
 (segment (start 150.3445 102.489) (end 151.003 102.489) (width 0.254) (layer F.Cu) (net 4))
 (segment (start 151.32999 105.22899) (end 152.146 106.045) (width 0.254) (layer F.Cu) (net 4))
 (segment (start 151.32999 102.81599) (end 151.32999 105.22899) (width 0.254) (layer F.Cu) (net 4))
 (segment (start 151.003 102.489) (end 151.32999 102.81599) (width 0.254) (layer F.Cu) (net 4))
 (segment (start 152.146 106.045) (end 149.606 106.045) (width 0.254) (layer B.Cu) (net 4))
 (segment (start 148.971 106.045) (end 148.59 106.426) (width 0.254) (layer F.Cu) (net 4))
 (segment (start 149.606 106.045) (end 148.971 106.045) (width 0.254) (layer F.Cu) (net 4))
 (segment (start 148.5075 100.311) (end 149.206 100.311) (width 0.254) (layer F.Cu) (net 3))
 (segment (start 149.352 100.457) (end 149.206 100.311) (width 0.254) (layer F.Cu) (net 3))
 (segment (start 150.3445 100.457) (end 149.352 100.457) (width 0.254) (layer F.Cu) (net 3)))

